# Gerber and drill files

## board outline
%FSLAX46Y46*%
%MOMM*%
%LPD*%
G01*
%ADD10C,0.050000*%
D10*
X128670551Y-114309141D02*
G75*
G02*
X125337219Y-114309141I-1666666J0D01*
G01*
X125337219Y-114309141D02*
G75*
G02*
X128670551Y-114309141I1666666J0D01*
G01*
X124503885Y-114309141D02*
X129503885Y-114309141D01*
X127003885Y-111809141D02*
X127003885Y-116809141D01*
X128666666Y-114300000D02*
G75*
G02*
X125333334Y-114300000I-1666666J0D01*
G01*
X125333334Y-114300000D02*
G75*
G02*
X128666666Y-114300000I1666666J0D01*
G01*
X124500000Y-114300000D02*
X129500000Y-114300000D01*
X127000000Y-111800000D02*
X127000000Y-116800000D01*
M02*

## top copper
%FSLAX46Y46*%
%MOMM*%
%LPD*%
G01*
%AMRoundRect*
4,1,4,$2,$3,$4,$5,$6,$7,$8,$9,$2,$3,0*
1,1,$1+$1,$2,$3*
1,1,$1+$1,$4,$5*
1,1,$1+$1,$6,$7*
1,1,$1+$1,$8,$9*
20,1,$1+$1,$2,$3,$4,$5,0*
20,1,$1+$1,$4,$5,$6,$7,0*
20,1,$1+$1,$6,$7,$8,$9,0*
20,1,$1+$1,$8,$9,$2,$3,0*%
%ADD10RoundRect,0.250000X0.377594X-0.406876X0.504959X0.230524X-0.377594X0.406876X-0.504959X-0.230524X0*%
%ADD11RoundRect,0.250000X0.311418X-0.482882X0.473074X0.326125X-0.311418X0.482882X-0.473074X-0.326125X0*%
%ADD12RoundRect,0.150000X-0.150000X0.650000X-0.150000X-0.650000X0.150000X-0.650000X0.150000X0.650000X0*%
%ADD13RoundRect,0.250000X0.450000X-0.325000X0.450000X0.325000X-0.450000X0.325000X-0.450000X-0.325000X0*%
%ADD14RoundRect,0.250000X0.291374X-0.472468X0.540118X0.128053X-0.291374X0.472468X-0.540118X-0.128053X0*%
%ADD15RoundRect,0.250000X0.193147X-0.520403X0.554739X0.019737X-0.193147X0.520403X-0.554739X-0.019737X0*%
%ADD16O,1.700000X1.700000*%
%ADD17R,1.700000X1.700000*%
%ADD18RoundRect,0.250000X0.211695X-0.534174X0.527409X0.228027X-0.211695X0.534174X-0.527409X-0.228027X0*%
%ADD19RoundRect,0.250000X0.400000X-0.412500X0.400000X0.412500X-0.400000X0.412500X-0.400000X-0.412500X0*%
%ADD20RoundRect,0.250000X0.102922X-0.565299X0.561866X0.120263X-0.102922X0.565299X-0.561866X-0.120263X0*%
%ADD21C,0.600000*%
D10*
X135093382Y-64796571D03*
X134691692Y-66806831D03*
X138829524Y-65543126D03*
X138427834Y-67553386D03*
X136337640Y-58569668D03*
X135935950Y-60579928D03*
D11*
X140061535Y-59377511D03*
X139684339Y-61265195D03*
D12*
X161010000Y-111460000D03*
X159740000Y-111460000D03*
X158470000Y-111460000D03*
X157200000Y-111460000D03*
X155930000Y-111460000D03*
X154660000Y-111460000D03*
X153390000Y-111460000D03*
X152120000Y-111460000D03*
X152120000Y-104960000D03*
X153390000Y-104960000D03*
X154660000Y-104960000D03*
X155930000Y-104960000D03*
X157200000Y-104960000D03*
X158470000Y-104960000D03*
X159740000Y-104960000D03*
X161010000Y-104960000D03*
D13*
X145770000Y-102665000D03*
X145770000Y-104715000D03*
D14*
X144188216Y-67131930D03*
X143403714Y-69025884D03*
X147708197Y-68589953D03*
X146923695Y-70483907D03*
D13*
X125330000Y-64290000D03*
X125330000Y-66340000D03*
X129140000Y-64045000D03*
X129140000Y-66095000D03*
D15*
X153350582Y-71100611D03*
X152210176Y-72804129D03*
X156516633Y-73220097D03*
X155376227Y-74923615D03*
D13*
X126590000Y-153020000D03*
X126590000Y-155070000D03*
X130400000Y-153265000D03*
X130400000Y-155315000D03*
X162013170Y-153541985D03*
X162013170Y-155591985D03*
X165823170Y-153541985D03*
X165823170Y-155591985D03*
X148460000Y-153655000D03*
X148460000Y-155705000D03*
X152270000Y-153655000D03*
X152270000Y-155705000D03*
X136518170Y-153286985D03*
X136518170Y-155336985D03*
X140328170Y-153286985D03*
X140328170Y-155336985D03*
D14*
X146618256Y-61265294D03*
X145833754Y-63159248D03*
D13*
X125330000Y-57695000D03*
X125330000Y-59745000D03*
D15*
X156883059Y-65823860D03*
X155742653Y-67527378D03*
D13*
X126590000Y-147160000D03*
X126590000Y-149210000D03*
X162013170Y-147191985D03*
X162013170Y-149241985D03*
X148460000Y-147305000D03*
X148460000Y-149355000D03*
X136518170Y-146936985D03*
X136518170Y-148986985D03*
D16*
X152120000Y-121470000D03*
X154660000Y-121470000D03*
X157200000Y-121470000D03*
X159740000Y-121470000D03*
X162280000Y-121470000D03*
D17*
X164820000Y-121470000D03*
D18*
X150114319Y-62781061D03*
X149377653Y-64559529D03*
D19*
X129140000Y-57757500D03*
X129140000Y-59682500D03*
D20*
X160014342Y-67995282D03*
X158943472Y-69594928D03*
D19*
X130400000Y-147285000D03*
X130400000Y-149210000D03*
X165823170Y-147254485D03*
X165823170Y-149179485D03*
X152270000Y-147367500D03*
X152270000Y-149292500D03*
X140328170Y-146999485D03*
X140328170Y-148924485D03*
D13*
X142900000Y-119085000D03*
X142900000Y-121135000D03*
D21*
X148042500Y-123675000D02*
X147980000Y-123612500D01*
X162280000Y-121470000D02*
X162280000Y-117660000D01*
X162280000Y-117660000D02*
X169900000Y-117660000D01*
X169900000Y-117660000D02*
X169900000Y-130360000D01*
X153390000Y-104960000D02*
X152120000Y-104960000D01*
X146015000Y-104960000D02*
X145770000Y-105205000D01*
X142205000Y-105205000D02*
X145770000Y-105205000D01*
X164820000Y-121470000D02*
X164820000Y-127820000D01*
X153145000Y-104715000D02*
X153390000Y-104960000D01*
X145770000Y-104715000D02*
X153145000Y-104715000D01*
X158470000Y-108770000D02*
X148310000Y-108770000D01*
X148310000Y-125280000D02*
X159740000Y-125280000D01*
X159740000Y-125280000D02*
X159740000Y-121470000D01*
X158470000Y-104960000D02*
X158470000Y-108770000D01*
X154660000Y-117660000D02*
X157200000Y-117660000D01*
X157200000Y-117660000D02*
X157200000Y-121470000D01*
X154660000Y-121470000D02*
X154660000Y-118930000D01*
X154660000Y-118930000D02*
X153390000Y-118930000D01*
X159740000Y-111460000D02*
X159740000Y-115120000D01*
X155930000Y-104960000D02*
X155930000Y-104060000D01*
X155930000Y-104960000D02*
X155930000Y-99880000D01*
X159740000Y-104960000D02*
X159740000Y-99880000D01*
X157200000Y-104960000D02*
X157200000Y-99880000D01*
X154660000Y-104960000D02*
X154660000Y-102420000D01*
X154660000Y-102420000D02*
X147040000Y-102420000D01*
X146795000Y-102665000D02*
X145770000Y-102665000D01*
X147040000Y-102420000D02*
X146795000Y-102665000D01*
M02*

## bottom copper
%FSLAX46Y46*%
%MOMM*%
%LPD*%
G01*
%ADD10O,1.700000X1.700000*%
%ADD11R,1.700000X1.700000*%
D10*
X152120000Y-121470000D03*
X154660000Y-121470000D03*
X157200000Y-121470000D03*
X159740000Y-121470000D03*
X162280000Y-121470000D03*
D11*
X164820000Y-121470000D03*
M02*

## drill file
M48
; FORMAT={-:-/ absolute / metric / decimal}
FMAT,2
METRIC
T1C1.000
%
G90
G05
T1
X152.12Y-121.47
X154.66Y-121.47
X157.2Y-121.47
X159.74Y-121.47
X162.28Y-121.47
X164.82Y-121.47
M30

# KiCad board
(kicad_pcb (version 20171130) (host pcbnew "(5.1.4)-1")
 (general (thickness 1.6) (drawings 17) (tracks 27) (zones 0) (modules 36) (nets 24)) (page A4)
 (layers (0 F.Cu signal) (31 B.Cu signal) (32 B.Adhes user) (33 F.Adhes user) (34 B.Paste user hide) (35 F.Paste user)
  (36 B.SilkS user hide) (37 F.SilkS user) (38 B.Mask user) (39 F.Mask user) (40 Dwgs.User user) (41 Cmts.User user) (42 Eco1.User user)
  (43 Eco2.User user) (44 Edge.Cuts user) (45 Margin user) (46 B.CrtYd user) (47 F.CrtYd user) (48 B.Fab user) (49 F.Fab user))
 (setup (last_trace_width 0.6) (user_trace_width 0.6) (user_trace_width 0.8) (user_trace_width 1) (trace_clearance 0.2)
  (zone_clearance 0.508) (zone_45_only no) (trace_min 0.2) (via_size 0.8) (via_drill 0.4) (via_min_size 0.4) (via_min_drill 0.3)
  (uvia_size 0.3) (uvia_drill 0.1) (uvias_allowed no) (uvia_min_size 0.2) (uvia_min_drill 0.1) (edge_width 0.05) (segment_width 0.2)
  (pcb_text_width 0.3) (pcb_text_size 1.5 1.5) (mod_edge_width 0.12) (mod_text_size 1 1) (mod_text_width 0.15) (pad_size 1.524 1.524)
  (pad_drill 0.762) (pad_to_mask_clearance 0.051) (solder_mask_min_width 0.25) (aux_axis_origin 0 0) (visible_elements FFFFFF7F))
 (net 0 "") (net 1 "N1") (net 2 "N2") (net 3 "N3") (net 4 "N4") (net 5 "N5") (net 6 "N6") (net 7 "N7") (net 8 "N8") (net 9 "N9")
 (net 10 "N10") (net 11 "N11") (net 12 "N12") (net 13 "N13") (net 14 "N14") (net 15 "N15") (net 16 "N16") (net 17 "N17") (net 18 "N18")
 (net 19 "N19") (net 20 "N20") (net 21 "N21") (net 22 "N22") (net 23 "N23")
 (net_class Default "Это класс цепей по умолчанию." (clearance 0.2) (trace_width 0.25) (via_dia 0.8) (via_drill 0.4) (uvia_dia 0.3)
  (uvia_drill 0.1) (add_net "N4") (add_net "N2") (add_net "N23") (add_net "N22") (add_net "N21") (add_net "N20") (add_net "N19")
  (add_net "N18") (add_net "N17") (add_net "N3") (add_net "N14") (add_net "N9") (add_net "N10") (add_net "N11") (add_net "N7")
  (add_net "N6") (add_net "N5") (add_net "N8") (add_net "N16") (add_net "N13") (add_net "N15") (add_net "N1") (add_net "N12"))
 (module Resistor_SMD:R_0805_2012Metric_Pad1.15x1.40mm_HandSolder (layer F.Cu) (at 134.892537 65.801701 78.7)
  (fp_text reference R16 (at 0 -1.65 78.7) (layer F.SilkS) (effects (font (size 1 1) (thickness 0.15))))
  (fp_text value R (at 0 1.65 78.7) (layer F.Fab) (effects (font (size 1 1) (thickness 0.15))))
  (pad 2 smd roundrect (at 1.025 0 78.7) (size 1.15 1.4) (layers F.Cu F.Paste F.Mask) (roundrect_rratio 0.217391) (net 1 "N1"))
  (pad 1 smd roundrect (at -1.025 0 78.7) (size 1.15 1.4) (layers F.Cu F.Paste F.Mask) (roundrect_rratio 0.217391) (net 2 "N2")))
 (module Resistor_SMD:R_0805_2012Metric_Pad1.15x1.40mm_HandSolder (layer F.Cu) (at 138.628679 66.548256 78.7)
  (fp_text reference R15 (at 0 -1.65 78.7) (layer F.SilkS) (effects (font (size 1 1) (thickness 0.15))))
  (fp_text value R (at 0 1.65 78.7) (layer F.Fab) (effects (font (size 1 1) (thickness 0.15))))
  (pad 2 smd roundrect (at 1.025 0 78.7) (size 1.15 1.4) (layers F.Cu F.Paste F.Mask) (roundrect_rratio 0.217391) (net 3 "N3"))
  (pad 1 smd roundrect (at -1.025 0 78.7) (size 1.15 1.4) (layers F.Cu F.Paste F.Mask) (roundrect_rratio 0.217391) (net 2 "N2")))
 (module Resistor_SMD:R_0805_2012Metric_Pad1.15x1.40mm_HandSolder (layer F.Cu) (at 136.136795 59.574798 78.7)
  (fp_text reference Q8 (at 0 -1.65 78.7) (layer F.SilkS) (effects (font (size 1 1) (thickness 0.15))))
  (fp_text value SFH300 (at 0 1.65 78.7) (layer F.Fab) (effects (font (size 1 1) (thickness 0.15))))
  (pad 2 smd roundrect (at 1.025 0 78.7) (size 1.15 1.4) (layers F.Cu F.Paste F.Mask) (roundrect_rratio 0.217391) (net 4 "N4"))
  (pad 1 smd roundrect (at -1.025 0 78.7) (size 1.15 1.4) (layers F.Cu F.Paste F.Mask) (roundrect_rratio 0.217391) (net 1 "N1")))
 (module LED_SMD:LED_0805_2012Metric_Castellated (layer F.Cu) (at 139.872937 60.321353 78.7)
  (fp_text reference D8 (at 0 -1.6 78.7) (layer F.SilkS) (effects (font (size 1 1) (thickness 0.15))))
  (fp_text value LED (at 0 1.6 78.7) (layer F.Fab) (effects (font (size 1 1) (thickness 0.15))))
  (pad 2 smd roundrect (at 0.9625 0 78.7) (size 1.325 1.3) (layers F.Cu F.Paste F.Mask) (roundrect_rratio 0.192308) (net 4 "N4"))
  (pad 1 smd roundrect (at -0.9625 0 78.7) (size 1.325 1.3) (layers F.Cu F.Paste F.Mask) (roundrect_rratio 0.192308) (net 3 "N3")))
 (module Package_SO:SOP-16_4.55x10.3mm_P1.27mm (layer F.Cu) (at 156.565 108.21 270)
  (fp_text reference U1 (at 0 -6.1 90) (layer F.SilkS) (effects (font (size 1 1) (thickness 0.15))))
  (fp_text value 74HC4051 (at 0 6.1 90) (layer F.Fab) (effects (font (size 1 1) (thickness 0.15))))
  (pad 16 smd roundrect (at 3.25 -4.445 270) (size 1.6 0.6) (layers F.Cu F.Paste F.Mask) (roundrect_rratio 0.25) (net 4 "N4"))
  (pad 15 smd roundrect (at 3.25 -3.175 270) (size 1.6 0.6) (layers F.Cu F.Paste F.Mask) (roundrect_rratio 0.25) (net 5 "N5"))
  (pad 14 smd roundrect (at 3.25 -1.905 270) (size 1.6 0.6) (layers F.Cu F.Paste F.Mask) (roundrect_rratio 0.25) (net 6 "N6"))
  (pad 13 smd roundrect (at 3.25 -0.635 270) (size 1.6 0.6) (layers F.Cu F.Paste F.Mask) (roundrect_rratio 0.25) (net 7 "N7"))
  (pad 12 smd roundrect (at 3.25 0.635 270) (size 1.6 0.6) (layers F.Cu F.Paste F.Mask) (roundrect_rratio 0.25) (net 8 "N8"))
  (pad 11 smd roundrect (at 3.25 1.905 270) (size 1.6 0.6) (layers F.Cu F.Paste F.Mask) (roundrect_rratio 0.25) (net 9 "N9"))
  (pad 10 smd roundrect (at 3.25 3.175 270) (size 1.6 0.6) (layers F.Cu F.Paste F.Mask) (roundrect_rratio 0.25) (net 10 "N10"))
  (pad 9 smd roundrect (at 3.25 4.445 270) (size 1.6 0.6) (layers F.Cu F.Paste F.Mask) (roundrect_rratio 0.25) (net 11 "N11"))
  (pad 8 smd roundrect (at -3.25 4.445 270) (size 1.6 0.6) (layers F.Cu F.Paste F.Mask) (roundrect_rratio 0.25) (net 2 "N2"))
  (pad 7 smd roundrect (at -3.25 3.175 270) (size 1.6 0.6) (layers F.Cu F.Paste F.Mask) (roundrect_rratio 0.25) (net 2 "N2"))
  (pad 6 smd roundrect (at -3.25 1.905 270) (size 1.6 0.6) (layers F.Cu F.Paste F.Mask) (roundrect_rratio 0.25) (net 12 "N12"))
  (pad 5 smd roundrect (at -3.25 0.635 270) (size 1.6 0.6) (layers F.Cu F.Paste F.Mask) (roundrect_rratio 0.25) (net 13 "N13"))
  (pad 4 smd roundrect (at -3.25 -0.635 270) (size 1.6 0.6) (layers F.Cu F.Paste F.Mask) (roundrect_rratio 0.25) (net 1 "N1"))
  (pad 3 smd roundrect (at -3.25 -1.905 270) (size 1.6 0.6) (layers F.Cu F.Paste F.Mask) (roundrect_rratio 0.25) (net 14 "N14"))
  (pad 2 smd roundrect (at -3.25 -3.175 270) (size 1.6 0.6) (layers F.Cu F.Paste F.Mask) (roundrect_rratio 0.25) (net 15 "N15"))
  (pad 1 smd roundrect (at -3.25 -4.445 270) (size 1.6 0.6) (layers F.Cu F.Paste F.Mask) (roundrect_rratio 0.25) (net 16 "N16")))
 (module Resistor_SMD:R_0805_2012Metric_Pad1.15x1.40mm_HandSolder (layer F.Cu) (at 145.77 103.69 90)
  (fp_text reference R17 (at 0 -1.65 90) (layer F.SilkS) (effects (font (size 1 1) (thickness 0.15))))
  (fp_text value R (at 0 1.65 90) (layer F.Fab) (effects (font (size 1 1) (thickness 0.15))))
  (pad 2 smd roundrect (at 1.025 0 90) (size 1.15 1.4) (layers F.Cu F.Paste F.Mask) (roundrect_rratio 0.217391) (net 12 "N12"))
  (pad 1 smd roundrect (at -1.025 0 90) (size 1.15 1.4) (layers F.Cu F.Paste F.Mask) (roundrect_rratio 0.217391) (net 2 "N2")))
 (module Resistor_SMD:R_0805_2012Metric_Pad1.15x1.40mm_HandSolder (layer F.Cu) (at 143.795965 68.078907 67.5)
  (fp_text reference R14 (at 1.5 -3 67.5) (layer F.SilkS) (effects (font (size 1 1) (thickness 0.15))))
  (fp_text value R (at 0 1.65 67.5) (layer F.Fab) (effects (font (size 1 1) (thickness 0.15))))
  (pad 2 smd roundrect (at 1.025 0 67.5) (size 1.15 1.4) (layers F.Cu F.Paste F.Mask) (roundrect_rratio 0.217391) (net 15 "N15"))
  (pad 1 smd roundrect (at -1.025 0 67.5) (size 1.15 1.4) (layers F.Cu F.Paste F.Mask) (roundrect_rratio 0.217391) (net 2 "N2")))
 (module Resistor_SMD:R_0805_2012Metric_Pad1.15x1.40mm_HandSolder (layer F.Cu) (at 147.315946 69.53693 67.5)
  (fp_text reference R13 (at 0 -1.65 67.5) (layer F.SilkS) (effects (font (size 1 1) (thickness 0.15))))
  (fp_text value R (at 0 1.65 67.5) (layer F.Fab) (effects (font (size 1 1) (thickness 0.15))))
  (pad 2 smd roundrect (at 1.025 0 67.5) (size 1.15 1.4) (layers F.Cu F.Paste F.Mask) (roundrect_rratio 0.217391) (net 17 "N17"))
  (pad 1 smd roundrect (at -1.025 0 67.5) (size 1.15 1.4) (layers F.Cu F.Paste F.Mask) (roundrect_rratio 0.217391) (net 2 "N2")))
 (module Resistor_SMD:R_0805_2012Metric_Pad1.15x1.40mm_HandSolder (layer F.Cu) (at 125.33 65.315 90)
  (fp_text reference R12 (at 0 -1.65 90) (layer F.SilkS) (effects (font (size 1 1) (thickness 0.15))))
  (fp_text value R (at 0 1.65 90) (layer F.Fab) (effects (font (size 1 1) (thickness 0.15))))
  (pad 2 smd roundrect (at 1.025 0 90) (size 1.15 1.4) (layers F.Cu F.Paste F.Mask) (roundrect_rratio 0.217391) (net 13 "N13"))
  (pad 1 smd roundrect (at -1.025 0 90) (size 1.15 1.4) (layers F.Cu F.Paste F.Mask) (roundrect_rratio 0.217391) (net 2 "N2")))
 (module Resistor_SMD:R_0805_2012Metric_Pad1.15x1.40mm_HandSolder (layer F.Cu) (at 129.14 65.07 90)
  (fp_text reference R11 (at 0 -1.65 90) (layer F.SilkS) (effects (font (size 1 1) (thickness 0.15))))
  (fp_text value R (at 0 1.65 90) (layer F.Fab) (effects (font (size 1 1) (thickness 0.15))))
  (pad 2 smd roundrect (at 1.025 0 90) (size 1.15 1.4) (layers F.Cu F.Paste F.Mask) (roundrect_rratio 0.217391) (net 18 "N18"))
  (pad 1 smd roundrect (at -1.025 0 90) (size 1.15 1.4) (layers F.Cu F.Paste F.Mask) (roundrect_rratio 0.217391) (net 2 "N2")))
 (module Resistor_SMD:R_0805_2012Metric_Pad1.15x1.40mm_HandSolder (layer F.Cu) (at 152.780379 71.95237 56.2)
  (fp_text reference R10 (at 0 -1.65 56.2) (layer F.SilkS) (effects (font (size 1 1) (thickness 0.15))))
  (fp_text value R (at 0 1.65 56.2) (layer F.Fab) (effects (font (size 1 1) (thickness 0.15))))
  (pad 2 smd roundrect (at 1.025 0 56.2) (size 1.15 1.4) (layers F.Cu F.Paste F.Mask) (roundrect_rratio 0.217391) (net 16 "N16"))
  (pad 1 smd roundrect (at -1.025 0 56.2) (size 1.15 1.4) (layers F.Cu F.Paste F.Mask) (roundrect_rratio 0.217391) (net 2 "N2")))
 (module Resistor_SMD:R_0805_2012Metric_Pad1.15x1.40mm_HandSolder (layer F.Cu) (at 155.94643 74.071856 56.2)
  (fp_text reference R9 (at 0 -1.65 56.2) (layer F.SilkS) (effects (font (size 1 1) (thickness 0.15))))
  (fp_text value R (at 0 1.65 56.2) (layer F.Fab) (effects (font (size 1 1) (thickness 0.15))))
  (pad 2 smd roundrect (at 1.025 0 56.2) (size 1.15 1.4) (layers F.Cu F.Paste F.Mask) (roundrect_rratio 0.217391) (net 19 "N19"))
  (pad 1 smd roundrect (at -1.025 0 56.2) (size 1.15 1.4) (layers F.Cu F.Paste F.Mask) (roundrect_rratio 0.217391) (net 2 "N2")))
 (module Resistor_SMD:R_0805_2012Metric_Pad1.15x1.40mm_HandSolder (layer F.Cu) (at 126.59 154.045 90)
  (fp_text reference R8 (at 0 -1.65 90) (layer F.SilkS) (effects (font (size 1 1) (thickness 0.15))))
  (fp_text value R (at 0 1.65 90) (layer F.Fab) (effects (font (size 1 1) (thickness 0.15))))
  (pad 2 smd roundrect (at 1.025 0 90) (size 1.15 1.4) (layers F.Cu F.Paste F.Mask) (roundrect_rratio 0.217391) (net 8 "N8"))
  (pad 1 smd roundrect (at -1.025 0 90) (size 1.15 1.4) (layers F.Cu F.Paste F.Mask) (roundrect_rratio 0.217391) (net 2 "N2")))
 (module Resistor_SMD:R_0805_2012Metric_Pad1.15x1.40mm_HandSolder (layer F.Cu) (at 130.4 154.29 90)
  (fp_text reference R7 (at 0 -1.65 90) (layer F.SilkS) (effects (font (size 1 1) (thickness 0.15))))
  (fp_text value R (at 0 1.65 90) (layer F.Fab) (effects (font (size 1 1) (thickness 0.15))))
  (pad 2 smd roundrect (at 1.025 0 90) (size 1.15 1.4) (layers F.Cu F.Paste F.Mask) (roundrect_rratio 0.217391) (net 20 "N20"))
  (pad 1 smd roundrect (at -1.025 0 90) (size 1.15 1.4) (layers F.Cu F.Paste F.Mask) (roundrect_rratio 0.217391) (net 2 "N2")))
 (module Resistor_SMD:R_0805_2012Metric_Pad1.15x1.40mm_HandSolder (layer F.Cu) (at 162.01317 154.566985 90)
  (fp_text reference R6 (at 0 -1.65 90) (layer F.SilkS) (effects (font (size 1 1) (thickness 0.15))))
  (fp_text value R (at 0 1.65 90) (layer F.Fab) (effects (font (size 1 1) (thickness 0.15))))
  (pad 2 smd roundrect (at 1.025 0 90) (size 1.15 1.4) (layers F.Cu F.Paste F.Mask) (roundrect_rratio 0.217391) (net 5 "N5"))
  (pad 1 smd roundrect (at -1.025 0 90) (size 1.15 1.4) (layers F.Cu F.Paste F.Mask) (roundrect_rratio 0.217391) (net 2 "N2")))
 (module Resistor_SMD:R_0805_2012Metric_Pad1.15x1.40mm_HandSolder (layer F.Cu) (at 165.82317 154.566985 90)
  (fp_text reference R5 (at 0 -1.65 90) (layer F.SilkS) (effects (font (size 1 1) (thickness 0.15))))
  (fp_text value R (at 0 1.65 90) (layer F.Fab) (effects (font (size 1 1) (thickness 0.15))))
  (pad 2 smd roundrect (at 1.025 0 90) (size 1.15 1.4) (layers F.Cu F.Paste F.Mask) (roundrect_rratio 0.217391) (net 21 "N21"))
  (pad 1 smd roundrect (at -1.025 0 90) (size 1.15 1.4) (layers F.Cu F.Paste F.Mask) (roundrect_rratio 0.217391) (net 2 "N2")))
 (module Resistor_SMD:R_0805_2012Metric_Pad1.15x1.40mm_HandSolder (layer F.Cu) (at 148.46 154.68 90)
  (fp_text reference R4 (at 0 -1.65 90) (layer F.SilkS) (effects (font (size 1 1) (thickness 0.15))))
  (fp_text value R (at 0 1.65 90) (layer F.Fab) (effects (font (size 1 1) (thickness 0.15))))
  (pad 2 smd roundrect (at 1.025 0 90) (size 1.15 1.4) (layers F.Cu F.Paste F.Mask) (roundrect_rratio 0.217391) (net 6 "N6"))
  (pad 1 smd roundrect (at -1.025 0 90) (size 1.15 1.4) (layers F.Cu F.Paste F.Mask) (roundrect_rratio 0.217391) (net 2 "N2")))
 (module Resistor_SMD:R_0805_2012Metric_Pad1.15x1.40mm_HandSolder (layer F.Cu) (at 152.27 154.68 90)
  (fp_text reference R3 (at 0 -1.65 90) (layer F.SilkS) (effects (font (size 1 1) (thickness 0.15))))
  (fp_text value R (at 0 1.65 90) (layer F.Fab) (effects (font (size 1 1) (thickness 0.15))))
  (pad 2 smd roundrect (at 1.025 0 90) (size 1.15 1.4) (layers F.Cu F.Paste F.Mask) (roundrect_rratio 0.217391) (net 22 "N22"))
  (pad 1 smd roundrect (at -1.025 0 90) (size 1.15 1.4) (layers F.Cu F.Paste F.Mask) (roundrect_rratio 0.217391) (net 2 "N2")))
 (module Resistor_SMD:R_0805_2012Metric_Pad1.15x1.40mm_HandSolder (layer F.Cu) (at 136.51817 154.311985 90)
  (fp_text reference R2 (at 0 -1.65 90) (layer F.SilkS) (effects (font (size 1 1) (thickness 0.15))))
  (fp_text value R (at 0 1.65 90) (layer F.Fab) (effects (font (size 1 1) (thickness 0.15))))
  (pad 2 smd roundrect (at 1.025 0 90) (size 1.15 1.4) (layers F.Cu F.Paste F.Mask) (roundrect_rratio 0.217391) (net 7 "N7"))
  (pad 1 smd roundrect (at -1.025 0 90) (size 1.15 1.4) (layers F.Cu F.Paste F.Mask) (roundrect_rratio 0.217391) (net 2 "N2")))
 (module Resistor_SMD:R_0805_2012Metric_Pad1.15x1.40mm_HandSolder (layer F.Cu) (at 140.32817 154.311985 90)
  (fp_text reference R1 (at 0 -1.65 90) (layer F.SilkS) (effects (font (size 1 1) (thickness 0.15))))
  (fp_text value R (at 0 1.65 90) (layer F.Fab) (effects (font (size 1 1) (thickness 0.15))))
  (pad 2 smd roundrect (at 1.025 0 90) (size 1.15 1.4) (layers F.Cu F.Paste F.Mask) (roundrect_rratio 0.217391) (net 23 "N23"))
  (pad 1 smd roundrect (at -1.025 0 90) (size 1.15 1.4) (layers F.Cu F.Paste F.Mask) (roundrect_rratio 0.217391) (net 2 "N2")))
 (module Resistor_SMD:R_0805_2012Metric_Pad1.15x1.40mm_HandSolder (layer F.Cu) (at 146.226005 62.212271 67.5)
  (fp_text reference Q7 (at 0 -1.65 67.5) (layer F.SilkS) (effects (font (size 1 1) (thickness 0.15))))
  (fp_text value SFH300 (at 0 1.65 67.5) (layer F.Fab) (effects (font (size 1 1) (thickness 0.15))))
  (pad 2 smd roundrect (at 1.025 0 67.5) (size 1.15 1.4) (layers F.Cu F.Paste F.Mask) (roundrect_rratio 0.217391) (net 4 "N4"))
  (pad 1 smd roundrect (at -1.025 0 67.5) (size 1.15 1.4) (layers F.Cu F.Paste F.Mask) (roundrect_rratio 0.217391) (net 15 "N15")))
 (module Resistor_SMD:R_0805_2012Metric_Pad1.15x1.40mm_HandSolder (layer F.Cu) (at 125.33 58.72 90)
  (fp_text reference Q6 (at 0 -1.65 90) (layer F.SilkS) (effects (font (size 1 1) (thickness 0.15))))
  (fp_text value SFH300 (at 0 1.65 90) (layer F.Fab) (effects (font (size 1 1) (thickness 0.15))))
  (pad 2 smd roundrect (at 1.025 0 90) (size 1.15 1.4) (layers F.Cu F.Paste F.Mask) (roundrect_rratio 0.217391) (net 4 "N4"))
  (pad 1 smd roundrect (at -1.025 0 90) (size 1.15 1.4) (layers F.Cu F.Paste F.Mask) (roundrect_rratio 0.217391) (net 13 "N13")))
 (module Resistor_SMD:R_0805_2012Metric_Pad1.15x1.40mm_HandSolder (layer F.Cu) (at 156.312856 66.675619 56.2)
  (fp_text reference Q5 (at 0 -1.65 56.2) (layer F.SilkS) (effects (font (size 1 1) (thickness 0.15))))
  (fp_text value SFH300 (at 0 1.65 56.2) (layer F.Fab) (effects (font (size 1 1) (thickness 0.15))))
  (pad 2 smd roundrect (at 1.025 0 56.2) (size 1.15 1.4) (layers F.Cu F.Paste F.Mask) (roundrect_rratio 0.217391) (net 4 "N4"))
  (pad 1 smd roundrect (at -1.025 0 56.2) (size 1.15 1.4) (layers F.Cu F.Paste F.Mask) (roundrect_rratio 0.217391) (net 16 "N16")))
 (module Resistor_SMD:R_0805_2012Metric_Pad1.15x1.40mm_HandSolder (layer F.Cu) (at 126.59 148.185 90)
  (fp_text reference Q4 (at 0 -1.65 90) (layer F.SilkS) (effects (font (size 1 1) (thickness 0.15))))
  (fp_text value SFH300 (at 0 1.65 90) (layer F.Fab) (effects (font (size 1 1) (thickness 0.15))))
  (pad 2 smd roundrect (at 1.025 0 90) (size 1.15 1.4) (layers F.Cu F.Paste F.Mask) (roundrect_rratio 0.217391) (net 4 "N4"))
  (pad 1 smd roundrect (at -1.025 0 90) (size 1.15 1.4) (layers F.Cu F.Paste F.Mask) (roundrect_rratio 0.217391) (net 8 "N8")))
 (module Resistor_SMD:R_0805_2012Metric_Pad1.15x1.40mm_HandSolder (layer F.Cu) (at 162.01317 148.216985 90)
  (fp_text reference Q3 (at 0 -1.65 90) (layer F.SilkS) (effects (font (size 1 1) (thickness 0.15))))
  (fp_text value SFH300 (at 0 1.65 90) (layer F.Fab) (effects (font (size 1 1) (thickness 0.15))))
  (pad 2 smd roundrect (at 1.025 0 90) (size 1.15 1.4) (layers F.Cu F.Paste F.Mask) (roundrect_rratio 0.217391) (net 4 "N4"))
  (pad 1 smd roundrect (at -1.025 0 90) (size 1.15 1.4) (layers F.Cu F.Paste F.Mask) (roundrect_rratio 0.217391) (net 5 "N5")))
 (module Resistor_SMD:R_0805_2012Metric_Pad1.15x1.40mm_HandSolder (layer F.Cu) (at 148.46 148.33 90)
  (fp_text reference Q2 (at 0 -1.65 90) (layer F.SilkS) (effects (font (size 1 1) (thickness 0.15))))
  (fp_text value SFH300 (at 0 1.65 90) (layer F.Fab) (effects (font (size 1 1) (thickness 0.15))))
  (pad 2 smd roundrect (at 1.025 0 90) (size 1.15 1.4) (layers F.Cu F.Paste F.Mask) (roundrect_rratio 0.217391) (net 4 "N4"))
  (pad 1 smd roundrect (at -1.025 0 90) (size 1.15 1.4) (layers F.Cu F.Paste F.Mask) (roundrect_rratio 0.217391) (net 6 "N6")))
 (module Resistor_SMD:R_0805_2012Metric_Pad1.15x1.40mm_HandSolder (layer F.Cu) (at 136.51817 147.961985 90)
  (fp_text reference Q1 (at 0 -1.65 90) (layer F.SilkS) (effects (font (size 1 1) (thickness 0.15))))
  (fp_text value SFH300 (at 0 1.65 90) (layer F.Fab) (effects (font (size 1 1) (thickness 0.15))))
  (pad 2 smd roundrect (at 1.025 0 90) (size 1.15 1.4) (layers F.Cu F.Paste F.Mask) (roundrect_rratio 0.217391) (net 4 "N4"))
  (pad 1 smd roundrect (at -1.025 0 90) (size 1.15 1.4) (layers F.Cu F.Paste F.Mask) (roundrect_rratio 0.217391) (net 7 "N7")))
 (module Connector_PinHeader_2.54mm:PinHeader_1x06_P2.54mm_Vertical (layer F.Cu) (at 164.82 121.47 270)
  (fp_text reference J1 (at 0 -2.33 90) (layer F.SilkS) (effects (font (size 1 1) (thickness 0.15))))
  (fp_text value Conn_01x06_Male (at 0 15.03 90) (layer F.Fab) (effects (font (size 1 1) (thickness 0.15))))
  (pad 6 thru_hole oval (at 0 12.7 270) (size 1.7 1.7) (drill 1) (layers *.Cu *.Mask) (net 11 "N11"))
  (pad 5 thru_hole oval (at 0 10.16 270) (size 1.7 1.7) (drill 1) (layers *.Cu *.Mask) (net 10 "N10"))
  (pad 4 thru_hole oval (at 0 7.62 270) (size 1.7 1.7) (drill 1) (layers *.Cu *.Mask) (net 9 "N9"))
  (pad 3 thru_hole oval (at 0 5.08 270) (size 1.7 1.7) (drill 1) (layers *.Cu *.Mask) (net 14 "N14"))
  (pad 2 thru_hole oval (at 0 2.54 270) (size 1.7 1.7) (drill 1) (layers *.Cu *.Mask) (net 4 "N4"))
  (pad 1 thru_hole rect (at 0 0 270) (size 1.7 1.7) (drill 1) (layers *.Cu *.Mask) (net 2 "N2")))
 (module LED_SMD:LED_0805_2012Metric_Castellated (layer F.Cu) (at 149.745986 63.670295 67.5)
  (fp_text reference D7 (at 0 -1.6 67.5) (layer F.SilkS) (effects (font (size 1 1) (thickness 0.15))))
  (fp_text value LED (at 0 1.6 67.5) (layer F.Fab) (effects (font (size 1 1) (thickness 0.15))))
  (pad 2 smd roundrect (at 0.9625 0 67.5) (size 1.325 1.3) (layers F.Cu F.Paste F.Mask) (roundrect_rratio 0.192308) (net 4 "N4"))
  (pad 1 smd roundrect (at -0.9625 0 67.5) (size 1.325 1.3) (layers F.Cu F.Paste F.Mask) (roundrect_rratio 0.192308) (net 17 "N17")))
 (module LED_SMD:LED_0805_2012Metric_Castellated (layer F.Cu) (at 129.14 58.72 90)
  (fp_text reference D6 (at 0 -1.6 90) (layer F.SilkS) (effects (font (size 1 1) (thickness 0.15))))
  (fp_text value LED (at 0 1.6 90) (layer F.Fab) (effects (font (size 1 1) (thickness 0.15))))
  (pad 2 smd roundrect (at 0.9625 0 90) (size 1.325 1.3) (layers F.Cu F.Paste F.Mask) (roundrect_rratio 0.192308) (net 4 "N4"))
  (pad 1 smd roundrect (at -0.9625 0 90) (size 1.325 1.3) (layers F.Cu F.Paste F.Mask) (roundrect_rratio 0.192308) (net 18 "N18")))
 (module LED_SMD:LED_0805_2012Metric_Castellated (layer F.Cu) (at 159.478907 68.795105 56.2)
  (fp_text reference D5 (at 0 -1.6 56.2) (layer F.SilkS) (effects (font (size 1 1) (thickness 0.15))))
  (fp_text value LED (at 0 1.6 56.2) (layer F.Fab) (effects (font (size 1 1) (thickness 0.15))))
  (pad 2 smd roundrect (at 0.9625 0 56.2) (size 1.325 1.3) (layers F.Cu F.Paste F.Mask) (roundrect_rratio 0.192308) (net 4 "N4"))
  (pad 1 smd roundrect (at -0.9625 0 56.2) (size 1.325 1.3) (layers F.Cu F.Paste F.Mask) (roundrect_rratio 0.192308) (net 19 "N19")))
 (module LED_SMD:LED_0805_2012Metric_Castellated (layer F.Cu) (at 130.4 148.2475 90)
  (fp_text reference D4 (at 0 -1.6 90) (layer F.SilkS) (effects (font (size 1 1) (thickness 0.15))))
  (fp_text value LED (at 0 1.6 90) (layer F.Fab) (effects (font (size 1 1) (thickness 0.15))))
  (pad 2 smd roundrect (at 0.9625 0 90) (size 1.325 1.3) (layers F.Cu F.Paste F.Mask) (roundrect_rratio 0.192308) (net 4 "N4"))
  (pad 1 smd roundrect (at -0.9625 0 90) (size 1.325 1.3) (layers F.Cu F.Paste F.Mask) (roundrect_rratio 0.192308) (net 20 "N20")))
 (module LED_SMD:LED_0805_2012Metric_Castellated (layer F.Cu) (at 165.82317 148.216985 90)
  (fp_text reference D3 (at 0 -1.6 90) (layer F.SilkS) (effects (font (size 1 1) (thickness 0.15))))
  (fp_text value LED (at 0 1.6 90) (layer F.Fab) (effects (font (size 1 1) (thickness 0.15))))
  (pad 2 smd roundrect (at 0.9625 0 90) (size 1.325 1.3) (layers F.Cu F.Paste F.Mask) (roundrect_rratio 0.192308) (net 4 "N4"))
  (pad 1 smd roundrect (at -0.9625 0 90) (size 1.325 1.3) (layers F.Cu F.Paste F.Mask) (roundrect_rratio 0.192308) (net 21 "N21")))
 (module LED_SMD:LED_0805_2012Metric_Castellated (layer F.Cu) (at 152.27 148.33 90)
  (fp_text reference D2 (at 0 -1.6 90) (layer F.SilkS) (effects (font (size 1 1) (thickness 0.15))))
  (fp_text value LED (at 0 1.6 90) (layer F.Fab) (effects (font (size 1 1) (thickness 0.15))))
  (pad 2 smd roundrect (at 0.9625 0 90) (size 1.325 1.3) (layers F.Cu F.Paste F.Mask) (roundrect_rratio 0.192308) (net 4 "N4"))
  (pad 1 smd roundrect (at -0.9625 0 90) (size 1.325 1.3) (layers F.Cu F.Paste F.Mask) (roundrect_rratio 0.192308) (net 22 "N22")))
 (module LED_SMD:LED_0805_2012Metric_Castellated (layer F.Cu) (at 140.32817 147.961985 90)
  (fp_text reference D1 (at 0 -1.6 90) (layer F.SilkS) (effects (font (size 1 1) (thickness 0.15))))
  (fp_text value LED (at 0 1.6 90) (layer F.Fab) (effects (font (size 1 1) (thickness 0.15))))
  (pad 2 smd roundrect (at 0.9625 0 90) (size 1.325 1.3) (layers F.Cu F.Paste F.Mask) (roundrect_rratio 0.192308) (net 4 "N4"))
  (pad 1 smd roundrect (at -0.9625 0 90) (size 1.325 1.3) (layers F.Cu F.Paste F.Mask) (roundrect_rratio 0.192308) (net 23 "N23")))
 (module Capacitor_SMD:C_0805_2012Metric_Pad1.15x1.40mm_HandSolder (layer F.Cu) (at 142.9 120.11 90)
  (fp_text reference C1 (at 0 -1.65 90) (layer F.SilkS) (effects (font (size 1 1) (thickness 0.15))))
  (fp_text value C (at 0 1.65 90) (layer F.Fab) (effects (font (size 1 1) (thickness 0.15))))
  (pad 2 smd roundrect (at 1.025 0 90) (size 1.15 1.4) (layers F.Cu F.Paste F.Mask) (roundrect_rratio 0.217391) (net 2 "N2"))
  (pad 1 smd roundrect (at -1.025 0 90) (size 1.15 1.4) (layers F.Cu F.Paste F.Mask) (roundrect_rratio 0.217391) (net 4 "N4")))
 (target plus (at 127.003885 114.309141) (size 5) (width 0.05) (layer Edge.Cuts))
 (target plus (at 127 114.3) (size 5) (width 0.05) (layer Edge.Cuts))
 (segment (start 148.0425 123.675) (end 147.98 123.6125) (width 0.6) (layer F.Cu) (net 4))
 (segment (start 162.28 121.47) (end 162.28 117.66) (width 0.6) (layer F.Cu) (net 4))
 (segment (start 162.28 117.66) (end 169.9 117.66) (width 0.6) (layer F.Cu) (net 4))
 (segment (start 169.9 117.66) (end 169.9 130.36) (width 0.6) (layer F.Cu) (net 4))
 (segment (start 153.39 104.96) (end 152.12 104.96) (width 0.6) (layer F.Cu) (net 2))
 (segment (start 146.015 104.96) (end 145.77 105.205) (width 0.6) (layer F.Cu) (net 2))
 (segment (start 142.205 105.205) (end 145.77 105.205) (width 0.6) (layer F.Cu) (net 2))
 (segment (start 164.82 121.47) (end 164.82 127.82) (width 0.6) (layer F.Cu) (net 2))
 (segment (start 153.145 104.715) (end 153.39 104.96) (width 0.6) (layer F.Cu) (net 2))
 (segment (start 145.77 104.715) (end 153.145 104.715) (width 0.6) (layer F.Cu) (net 2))
 (segment (start 158.47 108.77) (end 148.31 108.77) (width 0.6) (layer F.Cu) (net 14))
 (segment (start 148.31 125.28) (end 159.74 125.28) (width 0.6) (layer F.Cu) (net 14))
 (segment (start 159.74 125.28) (end 159.74 121.47) (width 0.6) (layer F.Cu) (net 14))
 (segment (start 158.47 104.96) (end 158.47 108.77) (width 0.6) (layer F.Cu) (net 14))
 (segment (start 154.66 117.66) (end 157.2 117.66) (width 0.6) (layer F.Cu) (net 9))
 (segment (start 157.2 117.66) (end 157.2 121.47) (width 0.6) (layer F.Cu) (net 9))
 (segment (start 154.66 121.47) (end 154.66 118.93) (width 0.6) (layer F.Cu) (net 10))
 (segment (start 154.66 118.93) (end 153.39 118.93) (width 0.6) (layer F.Cu) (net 10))
 (segment (start 159.74 111.46) (end 159.74 115.12) (width 0.6) (layer F.Cu) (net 5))
 (segment (start 155.93 104.96) (end 155.93 104.06) (width 0.6) (layer F.Cu) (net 13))
 (segment (start 155.93 104.96) (end 155.93 99.88) (width 0.6) (layer F.Cu) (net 13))
 (segment (start 159.74 104.96) (end 159.74 99.88) (width 0.6) (layer F.Cu) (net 15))
 (segment (start 157.2 104.96) (end 157.2 99.88) (width 0.6) (layer F.Cu) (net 1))
 (segment (start 154.66 104.96) (end 154.66 102.42) (width 0.6) (layer F.Cu) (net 12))
 (segment (start 154.66 102.42) (end 147.04 102.42) (width 0.6) (layer F.Cu) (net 12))
 (segment (start 146.795 102.665) (end 145.77 102.665) (width 0.6) (layer F.Cu) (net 12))
 (segment (start 147.04 102.42) (end 146.795 102.665) (width 0.6) (layer F.Cu) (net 12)))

